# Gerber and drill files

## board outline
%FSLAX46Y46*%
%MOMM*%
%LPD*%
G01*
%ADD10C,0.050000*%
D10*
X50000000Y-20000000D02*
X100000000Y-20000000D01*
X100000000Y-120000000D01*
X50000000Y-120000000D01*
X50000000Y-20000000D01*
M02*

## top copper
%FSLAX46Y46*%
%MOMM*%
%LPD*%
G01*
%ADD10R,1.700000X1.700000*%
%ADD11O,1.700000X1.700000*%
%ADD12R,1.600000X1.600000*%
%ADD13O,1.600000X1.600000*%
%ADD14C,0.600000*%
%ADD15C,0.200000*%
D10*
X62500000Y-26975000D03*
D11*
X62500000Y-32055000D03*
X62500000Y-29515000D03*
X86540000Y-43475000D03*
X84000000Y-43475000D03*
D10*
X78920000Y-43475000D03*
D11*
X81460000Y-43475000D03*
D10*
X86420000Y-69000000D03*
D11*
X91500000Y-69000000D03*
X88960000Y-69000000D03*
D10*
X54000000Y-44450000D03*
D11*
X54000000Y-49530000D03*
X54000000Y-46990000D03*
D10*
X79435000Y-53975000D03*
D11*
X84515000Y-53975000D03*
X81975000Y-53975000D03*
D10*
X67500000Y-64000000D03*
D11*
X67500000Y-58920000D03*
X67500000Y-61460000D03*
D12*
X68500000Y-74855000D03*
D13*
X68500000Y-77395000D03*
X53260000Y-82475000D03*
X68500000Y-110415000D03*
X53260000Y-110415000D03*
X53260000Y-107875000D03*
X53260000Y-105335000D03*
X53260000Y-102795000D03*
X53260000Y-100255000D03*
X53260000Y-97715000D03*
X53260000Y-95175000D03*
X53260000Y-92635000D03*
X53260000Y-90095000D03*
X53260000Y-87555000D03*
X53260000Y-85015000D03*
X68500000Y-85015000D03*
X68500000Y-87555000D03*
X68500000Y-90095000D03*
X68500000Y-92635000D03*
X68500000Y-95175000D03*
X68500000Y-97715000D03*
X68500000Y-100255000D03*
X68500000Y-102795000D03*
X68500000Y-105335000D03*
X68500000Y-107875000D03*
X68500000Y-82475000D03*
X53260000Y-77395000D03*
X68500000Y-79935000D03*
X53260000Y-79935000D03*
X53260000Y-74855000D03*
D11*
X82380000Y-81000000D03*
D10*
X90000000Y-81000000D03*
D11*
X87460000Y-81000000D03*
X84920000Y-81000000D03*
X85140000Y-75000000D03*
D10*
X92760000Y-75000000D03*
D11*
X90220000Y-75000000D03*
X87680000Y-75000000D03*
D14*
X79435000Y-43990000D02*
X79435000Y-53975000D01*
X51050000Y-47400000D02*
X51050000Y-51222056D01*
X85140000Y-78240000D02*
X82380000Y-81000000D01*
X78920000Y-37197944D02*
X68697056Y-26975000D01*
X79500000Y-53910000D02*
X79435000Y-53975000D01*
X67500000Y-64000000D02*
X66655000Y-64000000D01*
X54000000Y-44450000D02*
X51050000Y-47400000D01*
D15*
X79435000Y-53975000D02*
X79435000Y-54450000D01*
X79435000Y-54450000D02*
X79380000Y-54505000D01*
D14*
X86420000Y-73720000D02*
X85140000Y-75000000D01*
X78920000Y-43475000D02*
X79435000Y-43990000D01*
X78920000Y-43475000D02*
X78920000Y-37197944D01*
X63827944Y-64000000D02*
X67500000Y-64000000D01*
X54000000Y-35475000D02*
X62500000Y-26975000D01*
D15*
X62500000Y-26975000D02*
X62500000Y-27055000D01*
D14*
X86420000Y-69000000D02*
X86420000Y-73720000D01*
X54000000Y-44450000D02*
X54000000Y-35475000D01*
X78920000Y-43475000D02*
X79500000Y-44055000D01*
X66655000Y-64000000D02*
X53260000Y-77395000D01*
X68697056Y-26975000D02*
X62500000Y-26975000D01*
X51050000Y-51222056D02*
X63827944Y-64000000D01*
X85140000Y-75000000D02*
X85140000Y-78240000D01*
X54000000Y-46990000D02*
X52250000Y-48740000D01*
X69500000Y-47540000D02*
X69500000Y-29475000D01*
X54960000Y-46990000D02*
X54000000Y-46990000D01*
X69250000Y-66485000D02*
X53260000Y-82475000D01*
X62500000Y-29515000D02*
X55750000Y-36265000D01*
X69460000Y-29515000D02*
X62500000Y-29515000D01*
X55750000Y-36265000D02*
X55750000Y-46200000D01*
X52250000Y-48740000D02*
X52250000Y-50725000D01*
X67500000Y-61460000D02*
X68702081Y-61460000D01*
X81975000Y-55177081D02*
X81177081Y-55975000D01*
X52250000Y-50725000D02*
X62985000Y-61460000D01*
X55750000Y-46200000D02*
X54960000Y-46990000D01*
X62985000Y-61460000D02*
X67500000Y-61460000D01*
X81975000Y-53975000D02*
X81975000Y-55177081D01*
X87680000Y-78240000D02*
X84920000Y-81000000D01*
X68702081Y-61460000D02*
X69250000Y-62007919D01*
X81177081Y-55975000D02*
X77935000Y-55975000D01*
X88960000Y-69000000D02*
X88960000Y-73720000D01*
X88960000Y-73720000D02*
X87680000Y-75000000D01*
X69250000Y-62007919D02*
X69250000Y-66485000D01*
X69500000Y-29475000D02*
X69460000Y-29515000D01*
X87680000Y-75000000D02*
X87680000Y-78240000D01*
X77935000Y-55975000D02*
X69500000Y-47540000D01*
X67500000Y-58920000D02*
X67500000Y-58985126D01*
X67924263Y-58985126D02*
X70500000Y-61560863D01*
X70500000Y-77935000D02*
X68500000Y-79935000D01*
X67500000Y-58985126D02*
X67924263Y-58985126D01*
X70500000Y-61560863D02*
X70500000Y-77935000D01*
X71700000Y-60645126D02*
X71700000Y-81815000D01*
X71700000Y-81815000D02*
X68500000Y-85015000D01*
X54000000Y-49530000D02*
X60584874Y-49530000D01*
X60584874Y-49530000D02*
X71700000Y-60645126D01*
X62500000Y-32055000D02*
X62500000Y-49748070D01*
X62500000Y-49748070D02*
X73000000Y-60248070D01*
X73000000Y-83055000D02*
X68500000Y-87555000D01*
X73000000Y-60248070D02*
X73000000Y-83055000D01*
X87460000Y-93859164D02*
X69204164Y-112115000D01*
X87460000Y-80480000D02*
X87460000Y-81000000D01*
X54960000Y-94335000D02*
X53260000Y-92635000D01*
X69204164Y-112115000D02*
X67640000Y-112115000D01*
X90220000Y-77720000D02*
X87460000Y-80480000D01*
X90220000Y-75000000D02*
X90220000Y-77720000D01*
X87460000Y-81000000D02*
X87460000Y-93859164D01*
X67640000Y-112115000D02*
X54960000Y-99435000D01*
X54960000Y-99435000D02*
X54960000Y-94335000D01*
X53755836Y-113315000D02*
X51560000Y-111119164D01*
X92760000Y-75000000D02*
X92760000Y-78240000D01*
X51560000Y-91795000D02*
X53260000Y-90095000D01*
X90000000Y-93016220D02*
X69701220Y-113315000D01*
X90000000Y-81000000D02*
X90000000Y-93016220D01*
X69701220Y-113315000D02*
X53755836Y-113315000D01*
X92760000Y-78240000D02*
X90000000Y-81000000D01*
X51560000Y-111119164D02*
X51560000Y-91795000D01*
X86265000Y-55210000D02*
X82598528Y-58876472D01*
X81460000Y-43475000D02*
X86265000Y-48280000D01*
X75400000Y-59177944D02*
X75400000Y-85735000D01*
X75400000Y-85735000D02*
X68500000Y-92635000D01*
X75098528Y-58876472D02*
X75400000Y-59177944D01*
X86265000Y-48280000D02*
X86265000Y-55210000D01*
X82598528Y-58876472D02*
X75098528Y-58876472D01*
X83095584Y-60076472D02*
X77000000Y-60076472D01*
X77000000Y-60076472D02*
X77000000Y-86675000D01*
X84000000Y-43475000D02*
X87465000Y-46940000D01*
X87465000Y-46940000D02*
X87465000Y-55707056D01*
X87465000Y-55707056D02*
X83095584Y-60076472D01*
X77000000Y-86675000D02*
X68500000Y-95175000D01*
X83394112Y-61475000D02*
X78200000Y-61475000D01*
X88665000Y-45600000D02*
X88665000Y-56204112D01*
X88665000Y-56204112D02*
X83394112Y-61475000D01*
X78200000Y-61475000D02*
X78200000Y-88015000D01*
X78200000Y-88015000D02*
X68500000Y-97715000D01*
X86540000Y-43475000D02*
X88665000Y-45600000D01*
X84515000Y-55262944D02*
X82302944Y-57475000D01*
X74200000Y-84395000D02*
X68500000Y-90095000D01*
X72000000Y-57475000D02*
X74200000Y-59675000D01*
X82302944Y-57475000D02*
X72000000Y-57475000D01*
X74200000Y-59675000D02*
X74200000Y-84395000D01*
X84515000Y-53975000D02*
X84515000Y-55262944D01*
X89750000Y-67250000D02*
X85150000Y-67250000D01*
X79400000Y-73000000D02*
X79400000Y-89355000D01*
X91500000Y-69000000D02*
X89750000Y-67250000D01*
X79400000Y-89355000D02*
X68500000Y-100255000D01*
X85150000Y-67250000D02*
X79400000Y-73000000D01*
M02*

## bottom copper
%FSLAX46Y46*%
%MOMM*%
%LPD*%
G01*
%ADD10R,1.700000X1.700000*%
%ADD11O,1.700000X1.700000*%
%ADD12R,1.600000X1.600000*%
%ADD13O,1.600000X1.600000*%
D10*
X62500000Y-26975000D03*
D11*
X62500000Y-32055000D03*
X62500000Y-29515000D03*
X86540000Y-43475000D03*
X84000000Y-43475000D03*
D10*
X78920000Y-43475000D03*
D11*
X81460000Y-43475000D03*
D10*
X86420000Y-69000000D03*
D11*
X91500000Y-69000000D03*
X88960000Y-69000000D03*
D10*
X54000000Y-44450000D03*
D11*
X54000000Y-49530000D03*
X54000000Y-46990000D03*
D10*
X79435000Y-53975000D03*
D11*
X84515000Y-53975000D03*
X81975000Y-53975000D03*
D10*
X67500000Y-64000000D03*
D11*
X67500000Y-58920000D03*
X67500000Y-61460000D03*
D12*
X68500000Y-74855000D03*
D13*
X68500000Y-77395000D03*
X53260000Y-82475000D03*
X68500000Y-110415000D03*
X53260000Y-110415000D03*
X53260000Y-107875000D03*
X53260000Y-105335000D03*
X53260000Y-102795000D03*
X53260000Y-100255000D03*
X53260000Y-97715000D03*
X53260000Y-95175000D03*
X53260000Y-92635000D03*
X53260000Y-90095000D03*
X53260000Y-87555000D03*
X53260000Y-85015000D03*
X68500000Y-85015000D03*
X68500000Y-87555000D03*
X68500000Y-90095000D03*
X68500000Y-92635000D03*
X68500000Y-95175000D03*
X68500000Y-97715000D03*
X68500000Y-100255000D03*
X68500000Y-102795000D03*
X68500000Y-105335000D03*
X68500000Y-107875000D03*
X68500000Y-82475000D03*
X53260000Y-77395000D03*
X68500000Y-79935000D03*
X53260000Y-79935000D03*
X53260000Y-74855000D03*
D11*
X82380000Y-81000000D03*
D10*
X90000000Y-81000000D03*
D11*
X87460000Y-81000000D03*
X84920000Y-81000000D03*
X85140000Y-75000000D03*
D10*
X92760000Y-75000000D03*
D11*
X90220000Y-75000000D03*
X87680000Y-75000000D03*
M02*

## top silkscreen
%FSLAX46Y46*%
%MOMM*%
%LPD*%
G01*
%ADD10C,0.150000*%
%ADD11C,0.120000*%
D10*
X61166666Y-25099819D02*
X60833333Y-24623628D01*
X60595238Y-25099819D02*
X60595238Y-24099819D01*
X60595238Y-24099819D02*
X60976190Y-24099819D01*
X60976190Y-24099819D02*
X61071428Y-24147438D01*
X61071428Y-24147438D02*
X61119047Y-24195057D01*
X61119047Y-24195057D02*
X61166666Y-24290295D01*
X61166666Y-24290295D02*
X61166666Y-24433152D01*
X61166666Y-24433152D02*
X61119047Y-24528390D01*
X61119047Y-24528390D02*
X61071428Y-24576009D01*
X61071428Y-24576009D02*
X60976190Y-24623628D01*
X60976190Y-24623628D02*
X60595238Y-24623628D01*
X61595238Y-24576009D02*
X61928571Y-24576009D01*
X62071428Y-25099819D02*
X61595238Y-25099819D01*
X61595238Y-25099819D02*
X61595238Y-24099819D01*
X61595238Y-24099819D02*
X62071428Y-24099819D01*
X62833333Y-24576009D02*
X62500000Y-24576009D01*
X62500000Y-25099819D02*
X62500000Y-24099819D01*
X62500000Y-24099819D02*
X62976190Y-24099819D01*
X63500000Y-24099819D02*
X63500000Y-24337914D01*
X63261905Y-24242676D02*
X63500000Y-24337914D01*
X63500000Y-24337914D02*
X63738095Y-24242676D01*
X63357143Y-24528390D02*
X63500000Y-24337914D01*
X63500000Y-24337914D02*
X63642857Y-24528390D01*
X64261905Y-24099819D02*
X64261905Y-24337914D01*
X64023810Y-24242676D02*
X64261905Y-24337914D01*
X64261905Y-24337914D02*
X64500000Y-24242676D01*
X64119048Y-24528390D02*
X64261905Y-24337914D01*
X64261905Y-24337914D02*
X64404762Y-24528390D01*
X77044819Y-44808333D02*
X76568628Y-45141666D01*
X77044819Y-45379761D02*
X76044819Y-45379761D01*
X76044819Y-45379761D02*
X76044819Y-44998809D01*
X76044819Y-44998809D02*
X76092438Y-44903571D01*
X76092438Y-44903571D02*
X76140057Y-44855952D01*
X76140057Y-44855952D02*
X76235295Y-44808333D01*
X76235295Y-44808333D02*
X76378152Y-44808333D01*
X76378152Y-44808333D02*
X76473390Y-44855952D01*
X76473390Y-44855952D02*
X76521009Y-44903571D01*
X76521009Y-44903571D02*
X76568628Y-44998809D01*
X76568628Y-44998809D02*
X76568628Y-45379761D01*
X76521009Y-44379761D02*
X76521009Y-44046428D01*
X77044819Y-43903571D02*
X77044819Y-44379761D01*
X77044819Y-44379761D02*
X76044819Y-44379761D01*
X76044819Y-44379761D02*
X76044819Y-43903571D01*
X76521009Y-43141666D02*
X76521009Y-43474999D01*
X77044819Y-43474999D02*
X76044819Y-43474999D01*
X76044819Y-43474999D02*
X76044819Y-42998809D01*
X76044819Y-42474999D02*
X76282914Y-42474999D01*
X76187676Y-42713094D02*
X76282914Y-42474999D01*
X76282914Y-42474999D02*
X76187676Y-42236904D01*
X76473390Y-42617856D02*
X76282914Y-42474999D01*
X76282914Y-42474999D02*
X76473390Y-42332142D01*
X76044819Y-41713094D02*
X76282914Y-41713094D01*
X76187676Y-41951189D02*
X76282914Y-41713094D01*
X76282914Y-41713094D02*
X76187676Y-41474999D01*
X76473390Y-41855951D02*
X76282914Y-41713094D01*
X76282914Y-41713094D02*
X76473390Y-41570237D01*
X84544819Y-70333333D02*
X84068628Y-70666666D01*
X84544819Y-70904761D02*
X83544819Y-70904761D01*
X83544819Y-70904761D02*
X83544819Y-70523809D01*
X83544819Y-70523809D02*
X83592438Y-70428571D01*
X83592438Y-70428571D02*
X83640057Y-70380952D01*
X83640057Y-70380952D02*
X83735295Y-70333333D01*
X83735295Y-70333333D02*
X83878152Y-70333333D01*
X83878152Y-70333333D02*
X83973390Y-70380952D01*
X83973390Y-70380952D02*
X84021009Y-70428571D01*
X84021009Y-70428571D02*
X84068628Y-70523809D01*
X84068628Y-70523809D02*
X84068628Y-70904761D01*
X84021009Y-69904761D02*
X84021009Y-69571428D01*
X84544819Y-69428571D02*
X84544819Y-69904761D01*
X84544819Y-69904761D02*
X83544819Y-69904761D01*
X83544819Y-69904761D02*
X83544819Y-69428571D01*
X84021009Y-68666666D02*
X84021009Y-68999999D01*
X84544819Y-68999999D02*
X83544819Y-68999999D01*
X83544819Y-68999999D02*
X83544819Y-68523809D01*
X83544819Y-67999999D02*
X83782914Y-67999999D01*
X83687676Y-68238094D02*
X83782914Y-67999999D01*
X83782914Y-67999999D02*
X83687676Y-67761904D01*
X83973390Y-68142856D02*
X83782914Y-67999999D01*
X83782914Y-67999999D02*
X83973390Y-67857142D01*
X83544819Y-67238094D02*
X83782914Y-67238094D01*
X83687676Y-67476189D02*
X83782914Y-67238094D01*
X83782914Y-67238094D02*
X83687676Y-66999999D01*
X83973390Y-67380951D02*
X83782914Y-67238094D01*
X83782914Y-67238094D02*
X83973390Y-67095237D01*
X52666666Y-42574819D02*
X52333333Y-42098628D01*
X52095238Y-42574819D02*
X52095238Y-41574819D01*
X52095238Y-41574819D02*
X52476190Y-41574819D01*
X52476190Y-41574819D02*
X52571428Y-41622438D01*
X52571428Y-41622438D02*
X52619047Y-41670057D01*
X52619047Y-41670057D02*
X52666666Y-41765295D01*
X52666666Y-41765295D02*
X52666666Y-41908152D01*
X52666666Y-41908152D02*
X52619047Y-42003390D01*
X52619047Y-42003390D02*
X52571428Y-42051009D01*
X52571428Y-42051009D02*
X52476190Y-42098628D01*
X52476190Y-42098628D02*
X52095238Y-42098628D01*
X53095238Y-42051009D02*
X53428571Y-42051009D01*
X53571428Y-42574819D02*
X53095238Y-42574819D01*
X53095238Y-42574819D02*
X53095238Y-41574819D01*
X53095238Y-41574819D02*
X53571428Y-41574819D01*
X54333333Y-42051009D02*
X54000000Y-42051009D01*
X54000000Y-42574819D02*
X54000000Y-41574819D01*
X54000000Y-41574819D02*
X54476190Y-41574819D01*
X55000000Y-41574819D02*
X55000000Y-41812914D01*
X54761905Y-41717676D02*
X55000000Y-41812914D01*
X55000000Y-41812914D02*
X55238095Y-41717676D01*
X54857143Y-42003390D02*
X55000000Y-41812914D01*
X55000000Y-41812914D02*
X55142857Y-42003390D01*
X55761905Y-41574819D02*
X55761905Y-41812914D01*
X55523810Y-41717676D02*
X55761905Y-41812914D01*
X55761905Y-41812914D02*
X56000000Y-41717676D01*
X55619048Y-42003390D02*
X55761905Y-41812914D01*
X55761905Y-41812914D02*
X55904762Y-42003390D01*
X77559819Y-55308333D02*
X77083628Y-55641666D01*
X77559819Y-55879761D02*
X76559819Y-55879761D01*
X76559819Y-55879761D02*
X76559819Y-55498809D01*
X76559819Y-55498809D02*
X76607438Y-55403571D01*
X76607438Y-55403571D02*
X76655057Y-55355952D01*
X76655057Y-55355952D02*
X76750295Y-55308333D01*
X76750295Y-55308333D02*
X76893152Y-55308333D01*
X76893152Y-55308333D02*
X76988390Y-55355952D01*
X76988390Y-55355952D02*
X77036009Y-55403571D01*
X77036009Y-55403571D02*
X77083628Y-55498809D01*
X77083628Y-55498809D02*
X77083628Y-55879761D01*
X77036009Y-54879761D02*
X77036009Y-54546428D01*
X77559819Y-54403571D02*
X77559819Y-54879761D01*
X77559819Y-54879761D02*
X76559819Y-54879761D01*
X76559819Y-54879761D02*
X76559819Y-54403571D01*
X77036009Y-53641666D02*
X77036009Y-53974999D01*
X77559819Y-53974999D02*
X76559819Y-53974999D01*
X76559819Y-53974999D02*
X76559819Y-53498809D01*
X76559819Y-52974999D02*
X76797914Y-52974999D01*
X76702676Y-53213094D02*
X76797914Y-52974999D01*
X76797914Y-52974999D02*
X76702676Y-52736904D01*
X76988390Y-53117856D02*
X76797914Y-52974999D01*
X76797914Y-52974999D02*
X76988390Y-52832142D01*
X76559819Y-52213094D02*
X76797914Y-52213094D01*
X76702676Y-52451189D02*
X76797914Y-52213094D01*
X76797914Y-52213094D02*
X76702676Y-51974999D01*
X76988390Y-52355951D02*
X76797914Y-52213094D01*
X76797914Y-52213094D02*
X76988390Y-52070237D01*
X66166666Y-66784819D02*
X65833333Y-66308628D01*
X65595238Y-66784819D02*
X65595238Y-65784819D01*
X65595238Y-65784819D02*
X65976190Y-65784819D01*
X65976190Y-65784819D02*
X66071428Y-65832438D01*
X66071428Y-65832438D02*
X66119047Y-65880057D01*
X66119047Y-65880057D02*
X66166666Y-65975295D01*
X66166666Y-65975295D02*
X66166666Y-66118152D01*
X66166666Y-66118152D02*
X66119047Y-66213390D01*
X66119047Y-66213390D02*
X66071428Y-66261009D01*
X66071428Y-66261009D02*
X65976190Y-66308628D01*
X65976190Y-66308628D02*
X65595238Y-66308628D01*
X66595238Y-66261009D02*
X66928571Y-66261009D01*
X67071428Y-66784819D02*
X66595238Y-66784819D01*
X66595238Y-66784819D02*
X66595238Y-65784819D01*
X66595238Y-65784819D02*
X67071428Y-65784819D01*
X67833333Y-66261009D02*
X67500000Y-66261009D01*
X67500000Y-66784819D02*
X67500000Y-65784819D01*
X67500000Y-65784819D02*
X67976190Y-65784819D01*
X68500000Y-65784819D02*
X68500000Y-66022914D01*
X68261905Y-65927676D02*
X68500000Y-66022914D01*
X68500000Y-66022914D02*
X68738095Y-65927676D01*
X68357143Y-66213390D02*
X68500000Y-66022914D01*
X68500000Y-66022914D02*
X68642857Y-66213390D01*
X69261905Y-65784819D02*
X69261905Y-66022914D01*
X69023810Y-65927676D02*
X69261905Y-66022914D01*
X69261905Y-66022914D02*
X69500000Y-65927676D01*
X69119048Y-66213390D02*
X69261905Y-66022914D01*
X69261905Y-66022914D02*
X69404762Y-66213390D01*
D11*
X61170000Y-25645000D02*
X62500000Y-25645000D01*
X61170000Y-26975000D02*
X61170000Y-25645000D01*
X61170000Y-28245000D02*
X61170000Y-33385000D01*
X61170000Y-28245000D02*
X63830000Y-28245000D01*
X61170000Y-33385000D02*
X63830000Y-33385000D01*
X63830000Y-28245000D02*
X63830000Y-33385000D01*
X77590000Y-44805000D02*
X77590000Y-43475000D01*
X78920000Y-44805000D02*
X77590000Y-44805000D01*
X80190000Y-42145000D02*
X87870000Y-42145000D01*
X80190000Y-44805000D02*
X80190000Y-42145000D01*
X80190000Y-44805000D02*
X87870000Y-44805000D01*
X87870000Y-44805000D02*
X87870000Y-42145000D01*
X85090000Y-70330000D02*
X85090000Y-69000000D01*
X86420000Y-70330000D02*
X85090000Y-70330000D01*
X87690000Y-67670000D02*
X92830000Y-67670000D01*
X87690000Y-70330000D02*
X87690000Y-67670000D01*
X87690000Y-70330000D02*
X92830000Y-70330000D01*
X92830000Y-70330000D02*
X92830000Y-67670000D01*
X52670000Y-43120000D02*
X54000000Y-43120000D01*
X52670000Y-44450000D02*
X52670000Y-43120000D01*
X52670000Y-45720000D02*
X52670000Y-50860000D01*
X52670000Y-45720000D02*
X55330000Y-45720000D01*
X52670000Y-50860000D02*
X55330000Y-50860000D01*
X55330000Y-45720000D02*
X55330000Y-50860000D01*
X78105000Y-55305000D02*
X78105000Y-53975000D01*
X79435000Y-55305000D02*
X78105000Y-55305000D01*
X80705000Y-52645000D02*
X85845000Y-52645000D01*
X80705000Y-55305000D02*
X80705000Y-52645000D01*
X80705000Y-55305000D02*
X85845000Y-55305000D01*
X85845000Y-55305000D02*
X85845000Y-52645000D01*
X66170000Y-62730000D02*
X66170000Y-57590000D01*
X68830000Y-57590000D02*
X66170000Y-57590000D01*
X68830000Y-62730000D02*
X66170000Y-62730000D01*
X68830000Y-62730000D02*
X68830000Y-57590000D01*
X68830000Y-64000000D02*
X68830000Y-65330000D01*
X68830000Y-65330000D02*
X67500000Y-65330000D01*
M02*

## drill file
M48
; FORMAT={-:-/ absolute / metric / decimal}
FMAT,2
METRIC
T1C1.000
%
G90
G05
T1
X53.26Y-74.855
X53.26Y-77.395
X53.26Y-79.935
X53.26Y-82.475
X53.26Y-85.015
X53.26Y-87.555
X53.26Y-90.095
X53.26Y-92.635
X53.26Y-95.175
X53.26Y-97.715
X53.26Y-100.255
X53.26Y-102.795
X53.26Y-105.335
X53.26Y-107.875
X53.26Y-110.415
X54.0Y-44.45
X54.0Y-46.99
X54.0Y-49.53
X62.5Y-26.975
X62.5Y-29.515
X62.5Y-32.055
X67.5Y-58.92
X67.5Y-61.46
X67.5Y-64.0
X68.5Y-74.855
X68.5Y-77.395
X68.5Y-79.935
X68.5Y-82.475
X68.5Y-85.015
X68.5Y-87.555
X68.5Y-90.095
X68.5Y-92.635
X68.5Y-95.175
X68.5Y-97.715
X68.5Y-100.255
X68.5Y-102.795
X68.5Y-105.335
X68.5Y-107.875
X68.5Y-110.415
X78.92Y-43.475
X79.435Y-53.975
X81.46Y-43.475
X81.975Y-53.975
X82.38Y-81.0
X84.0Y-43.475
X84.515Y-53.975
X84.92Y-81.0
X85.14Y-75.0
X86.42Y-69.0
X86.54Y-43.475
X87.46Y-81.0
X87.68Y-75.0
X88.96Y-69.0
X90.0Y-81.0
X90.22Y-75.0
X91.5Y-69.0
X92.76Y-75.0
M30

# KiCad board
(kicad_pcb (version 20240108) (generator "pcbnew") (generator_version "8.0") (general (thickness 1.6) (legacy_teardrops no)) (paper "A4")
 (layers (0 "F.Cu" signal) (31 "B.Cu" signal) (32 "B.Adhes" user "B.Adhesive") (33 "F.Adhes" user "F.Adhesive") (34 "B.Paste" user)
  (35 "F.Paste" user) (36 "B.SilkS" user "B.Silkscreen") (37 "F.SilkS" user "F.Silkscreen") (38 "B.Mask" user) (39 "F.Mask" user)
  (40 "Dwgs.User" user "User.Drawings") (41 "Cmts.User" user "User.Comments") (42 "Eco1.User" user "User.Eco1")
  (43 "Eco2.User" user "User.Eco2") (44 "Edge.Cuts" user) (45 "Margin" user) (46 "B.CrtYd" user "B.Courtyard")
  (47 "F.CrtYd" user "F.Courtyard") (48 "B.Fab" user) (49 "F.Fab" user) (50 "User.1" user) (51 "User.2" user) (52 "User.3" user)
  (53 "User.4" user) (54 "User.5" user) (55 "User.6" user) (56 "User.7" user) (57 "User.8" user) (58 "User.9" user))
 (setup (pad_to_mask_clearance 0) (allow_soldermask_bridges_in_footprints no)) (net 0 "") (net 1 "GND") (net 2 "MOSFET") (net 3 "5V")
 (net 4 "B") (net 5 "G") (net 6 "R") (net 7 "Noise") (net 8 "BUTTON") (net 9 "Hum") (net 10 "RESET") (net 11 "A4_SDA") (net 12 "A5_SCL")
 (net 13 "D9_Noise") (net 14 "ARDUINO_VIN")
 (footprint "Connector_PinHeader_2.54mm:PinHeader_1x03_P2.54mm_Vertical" (layer "F.Cu") (at 62.5 26.975)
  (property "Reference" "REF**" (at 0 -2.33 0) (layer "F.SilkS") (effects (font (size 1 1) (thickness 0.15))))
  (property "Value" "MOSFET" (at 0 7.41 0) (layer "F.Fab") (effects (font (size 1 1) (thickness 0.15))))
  (fp_line (start -1.33 -1.33) (end 0 -1.33) (stroke (width 0.12) (type solid)) (layer "F.SilkS"))
  (fp_line (start -1.33 0) (end -1.33 -1.33) (stroke (width 0.12) (type solid)) (layer "F.SilkS"))
  (fp_line (start -1.33 1.27) (end -1.33 6.41) (stroke (width 0.12) (type solid)) (layer "F.SilkS"))
  (fp_line (start -1.33 1.27) (end 1.33 1.27) (stroke (width 0.12) (type solid)) (layer "F.SilkS"))
  (fp_line (start -1.33 6.41) (end 1.33 6.41) (stroke (width 0.12) (type solid)) (layer "F.SilkS"))
  (fp_line (start 1.33 1.27) (end 1.33 6.41) (stroke (width 0.12) (type solid)) (layer "F.SilkS"))
  (pad "GND" thru_hole rect (at 0 0) (size 1.7 1.7) (drill 1) (layers "*.Cu" "*.Mask") (remove_unused_layers no) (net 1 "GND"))
  (pad "S" thru_hole oval (at 0 5.08) (size 1.7 1.7) (drill 1) (layers "*.Cu" "*.Mask") (remove_unused_layers no) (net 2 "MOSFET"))
  (pad "VCC" thru_hole oval (at 0 2.54) (size 1.7 1.7) (drill 1) (layers "*.Cu" "*.Mask") (remove_unused_layers no) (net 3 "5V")))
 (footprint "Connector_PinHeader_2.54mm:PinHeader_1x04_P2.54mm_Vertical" (layer "F.Cu") (at 78.92 43.475 90)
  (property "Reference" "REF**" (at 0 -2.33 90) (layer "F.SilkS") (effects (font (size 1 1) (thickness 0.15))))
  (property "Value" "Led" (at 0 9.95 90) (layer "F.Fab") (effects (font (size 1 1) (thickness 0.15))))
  (fp_line (start -1.33 -1.33) (end 0 -1.33) (stroke (width 0.12) (type solid)) (layer "F.SilkS"))
  (fp_line (start -1.33 0) (end -1.33 -1.33) (stroke (width 0.12) (type solid)) (layer "F.SilkS"))
  (fp_line (start 1.33 1.27) (end 1.33 8.95) (stroke (width 0.12) (type solid)) (layer "F.SilkS"))
  (fp_line (start -1.33 1.27) (end 1.33 1.27) (stroke (width 0.12) (type solid)) (layer "F.SilkS"))
  (fp_line (start -1.33 1.27) (end -1.33 8.95) (stroke (width 0.12) (type solid)) (layer "F.SilkS"))
  (fp_line (start -1.33 8.95) (end 1.33 8.95) (stroke (width 0.12) (type solid)) (layer "F.SilkS"))
  (pad "B" thru_hole oval (at 0 7.62 90) (size 1.7 1.7) (drill 1) (layers "*.Cu" "*.Mask") (remove_unused_layers no) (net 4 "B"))
  (pad "G" thru_hole oval (at 0 5.08 90) (size 1.7 1.7) (drill 1) (layers "*.Cu" "*.Mask") (remove_unused_layers no) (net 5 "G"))
  (pad "GND" thru_hole rect (at 0 0 90) (size 1.7 1.7) (drill 1) (layers "*.Cu" "*.Mask") (remove_unused_layers no) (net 1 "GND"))
  (pad "R" thru_hole oval (at 0 2.54 90) (size 1.7 1.7) (drill 1) (layers "*.Cu" "*.Mask") (remove_unused_layers no) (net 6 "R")))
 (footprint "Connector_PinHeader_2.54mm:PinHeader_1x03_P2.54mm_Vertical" (layer "F.Cu") (at 86.42 69 90)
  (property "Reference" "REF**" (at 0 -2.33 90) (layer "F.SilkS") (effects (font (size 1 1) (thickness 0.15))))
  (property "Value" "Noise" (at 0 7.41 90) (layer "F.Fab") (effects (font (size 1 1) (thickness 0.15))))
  (fp_line (start -1.33 -1.33) (end 0 -1.33) (stroke (width 0.12) (type solid)) (layer "F.SilkS"))
  (fp_line (start -1.33 0) (end -1.33 -1.33) (stroke (width 0.12) (type solid)) (layer "F.SilkS"))
  (fp_line (start 1.33 1.27) (end 1.33 6.41) (stroke (width 0.12) (type solid)) (layer "F.SilkS"))
  (fp_line (start -1.33 1.27) (end 1.33 1.27) (stroke (width 0.12) (type solid)) (layer "F.SilkS"))
  (fp_line (start -1.33 1.27) (end -1.33 6.41) (stroke (width 0.12) (type solid)) (layer "F.SilkS"))
  (fp_line (start -1.33 6.41) (end 1.33 6.41) (stroke (width 0.12) (type solid)) (layer "F.SilkS"))
  (pad "GND" thru_hole rect (at 0 0 90) (size 1.7 1.7) (drill 1) (layers "*.Cu" "*.Mask") (remove_unused_layers no) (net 1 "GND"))
  (pad "S" thru_hole oval (at 0 5.08 90) (size 1.7 1.7) (drill 1) (layers "*.Cu" "*.Mask") (remove_unused_layers no) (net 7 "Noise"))
  (pad "VCC" thru_hole oval (at 0 2.54 90) (size 1.7 1.7) (drill 1) (layers "*.Cu" "*.Mask") (remove_unused_layers no) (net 3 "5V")))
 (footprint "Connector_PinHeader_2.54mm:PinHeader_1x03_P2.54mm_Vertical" (layer "F.Cu") (at 54 44.45)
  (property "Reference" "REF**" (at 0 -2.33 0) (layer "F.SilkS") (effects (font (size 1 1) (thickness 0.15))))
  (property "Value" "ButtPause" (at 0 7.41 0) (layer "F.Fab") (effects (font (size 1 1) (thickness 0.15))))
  (fp_line (start -1.33 -1.33) (end 0 -1.33) (stroke (width 0.12) (type solid)) (layer "F.SilkS"))
  (fp_line (start -1.33 0) (end -1.33 -1.33) (stroke (width 0.12) (type solid)) (layer "F.SilkS"))
  (fp_line (start -1.33 1.27) (end -1.33 6.41) (stroke (width 0.12) (type solid)) (layer "F.SilkS"))
  (fp_line (start -1.33 1.27) (end 1.33 1.27) (stroke (width 0.12) (type solid)) (layer "F.SilkS"))
  (fp_line (start -1.33 6.41) (end 1.33 6.41) (stroke (width 0.12) (type solid)) (layer "F.SilkS"))
  (fp_line (start 1.33 1.27) (end 1.33 6.41) (stroke (width 0.12) (type solid)) (layer "F.SilkS"))
  (pad "GND" thru_hole rect (at 0 0) (size 1.7 1.7) (drill 1) (layers "*.Cu" "*.Mask") (remove_unused_layers no) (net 1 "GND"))
  (pad "S" thru_hole oval (at 0 5.08) (size 1.7 1.7) (drill 1) (layers "*.Cu" "*.Mask") (remove_unused_layers no) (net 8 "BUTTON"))
  (pad "VCC" thru_hole oval (at 0 2.54) (size 1.7 1.7) (drill 1) (layers "*.Cu" "*.Mask") (remove_unused_layers no) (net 3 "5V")))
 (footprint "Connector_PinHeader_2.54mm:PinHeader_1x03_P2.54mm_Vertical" (layer "F.Cu") (at 79.435 53.975 90)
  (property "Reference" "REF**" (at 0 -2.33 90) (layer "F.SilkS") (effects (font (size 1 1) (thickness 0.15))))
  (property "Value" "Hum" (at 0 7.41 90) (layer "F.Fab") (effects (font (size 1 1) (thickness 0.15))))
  (fp_line (start -1.33 -1.33) (end 0 -1.33) (stroke (width 0.12) (type solid)) (layer "F.SilkS"))
  (fp_line (start -1.33 0) (end -1.33 -1.33) (stroke (width 0.12) (type solid)) (layer "F.SilkS"))
  (fp_line (start 1.33 1.27) (end 1.33 6.41) (stroke (width 0.12) (type solid)) (layer "F.SilkS"))
  (fp_line (start -1.33 1.27) (end 1.33 1.27) (stroke (width 0.12) (type solid)) (layer "F.SilkS"))
  (fp_line (start -1.33 1.27) (end -1.33 6.41) (stroke (width 0.12) (type solid)) (layer "F.SilkS"))
  (fp_line (start -1.33 6.41) (end 1.33 6.41) (stroke (width 0.12) (type solid)) (layer "F.SilkS"))
  (pad "GND" thru_hole rect (at 0 0 90) (size 1.7 1.7) (drill 1) (layers "*.Cu" "*.Mask") (remove_unused_layers no) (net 1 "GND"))
  (pad "S" thru_hole oval (at 0 5.08 90) (size 1.7 1.7) (drill 1) (layers "*.Cu" "*.Mask") (remove_unused_layers no) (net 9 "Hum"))
  (pad "VCC" thru_hole oval (at 0 2.54 90) (size 1.7 1.7) (drill 1) (layers "*.Cu" "*.Mask") (remove_unused_layers no) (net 3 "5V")))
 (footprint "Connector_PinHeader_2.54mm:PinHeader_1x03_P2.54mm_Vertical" (layer "F.Cu") (at 67.5 64 180)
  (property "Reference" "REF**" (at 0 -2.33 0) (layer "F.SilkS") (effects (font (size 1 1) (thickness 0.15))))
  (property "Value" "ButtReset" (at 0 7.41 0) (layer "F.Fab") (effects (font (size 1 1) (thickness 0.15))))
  (fp_line (start 1.33 1.27) (end 1.33 6.41) (stroke (width 0.12) (type solid)) (layer "F.SilkS"))
  (fp_line (start -1.33 6.41) (end 1.33 6.41) (stroke (width 0.12) (type solid)) (layer "F.SilkS"))
  (fp_line (start -1.33 1.27) (end 1.33 1.27) (stroke (width 0.12) (type solid)) (layer "F.SilkS"))
  (fp_line (start -1.33 1.27) (end -1.33 6.41) (stroke (width 0.12) (type solid)) (layer "F.SilkS"))
  (fp_line (start -1.33 0) (end -1.33 -1.33) (stroke (width 0.12) (type solid)) (layer "F.SilkS"))
  (fp_line (start -1.33 -1.33) (end 0 -1.33) (stroke (width 0.12) (type solid)) (layer "F.SilkS"))
  (pad "GND" thru_hole rect (at 0 0 180) (size 1.7 1.7) (drill 1) (layers "*.Cu" "*.Mask") (remove_unused_layers no) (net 1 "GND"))
  (pad "S" thru_hole oval (at 0 5.08 180) (size 1.7 1.7) (drill 1) (layers "*.Cu" "*.Mask") (remove_unused_layers no) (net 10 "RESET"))
  (pad "VCC" thru_hole oval (at 0 2.54 180) (size 1.7 1.7) (drill 1) (layers "*.Cu" "*.Mask") (remove_unused_layers no) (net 3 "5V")))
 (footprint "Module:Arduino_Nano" (layer "B.Cu") (at 68.5 74.855 180)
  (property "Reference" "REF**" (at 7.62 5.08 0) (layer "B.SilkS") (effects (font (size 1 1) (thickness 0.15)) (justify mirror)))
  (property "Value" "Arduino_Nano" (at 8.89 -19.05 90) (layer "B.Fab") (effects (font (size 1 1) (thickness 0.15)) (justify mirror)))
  (pad "1" thru_hole rect (at 0 0 180) (size 1.6 1.6) (drill 1) (layers "*.Cu" "*.Mask") (remove_unused_layers no))
  (pad "2" thru_hole oval (at 0 -2.54 180) (size 1.6 1.6) (drill 1) (layers "*.Cu" "*.Mask") (remove_unused_layers no))
  (pad "5V" thru_hole oval (at 15.24 -7.62 180) (size 1.6 1.6) (drill 1) (layers "*.Cu" "*.Mask") (remove_unused_layers no) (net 3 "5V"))
  (pad "15" thru_hole oval (at 0 -35.56 180) (size 1.6 1.6) (drill 1) (layers "*.Cu" "*.Mask") (remove_unused_layers no))
  (pad "16" thru_hole oval (at 15.24 -35.56 180) (size 1.6 1.6) (drill 1) (layers "*.Cu" "*.Mask") (remove_unused_layers no))
  (pad "17" thru_hole oval (at 15.24 -33.02 180) (size 1.6 1.6) (drill 1) (layers "*.Cu" "*.Mask") (remove_unused_layers no))
  (pad "18" thru_hole oval (at 15.24 -30.48 180) (size 1.6 1.6) (drill 1) (layers "*.Cu" "*.Mask") (remove_unused_layers no))
  (pad "A0" thru_hole oval (at 15.24 -27.94 180) (size 1.6 1.6) (drill 1) (layers "*.Cu" "*.Mask") (remove_unused_layers no))
  (pad "A1" thru_hole oval (at 15.24 -25.4 180) (size 1.6 1.6) (drill 1) (layers "*.Cu" "*.Mask") (remove_unused_layers no))
  (pad "A2" thru_hole oval (at 15.24 -22.86 180) (size 1.6 1.6) (drill 1) (layers "*.Cu" "*.Mask") (remove_unused_layers no))
  (pad "A3" thru_hole oval (at 15.24 -20.32 180) (size 1.6 1.6) (drill 1) (layers "*.Cu" "*.Mask") (remove_unused_layers no))
  (pad "A4" thru_hole oval (at 15.24 -17.78 180) (size 1.6 1.6) (drill 1) (layers "*.Cu" "*.Mask") (remove_unused_layers no)
   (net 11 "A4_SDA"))
  (pad "A5" thru_hole oval (at 15.24 -15.24 180) (size 1.6 1.6) (drill 1) (layers "*.Cu" "*.Mask") (remove_unused_layers no)
   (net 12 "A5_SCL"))
  (pad "A6" thru_hole oval (at 15.24 -12.7 180) (size 1.6 1.6) (drill 1) (layers "*.Cu" "*.Mask") (remove_unused_layers no))
  (pad "A7" thru_hole oval (at 15.24 -10.16 180) (size 1.6 1.6) (drill 1) (layers "*.Cu" "*.Mask") (remove_unused_layers no))
  (pad "D2" thru_hole oval (at 0 -10.16 180) (size 1.6 1.6) (drill 1) (layers "*.Cu" "*.Mask") (remove_unused_layers no) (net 8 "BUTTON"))
  (pad "D3" thru_hole oval (at 0 -12.7 180) (size 1.6 1.6) (drill 1) (layers "*.Cu" "*.Mask") (remove_unused_layers no) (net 2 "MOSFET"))
  (pad "D4" thru_hole oval (at 0 -15.24 180) (size 1.6 1.6) (drill 1) (layers "*.Cu" "*.Mask") (remove_unused_layers no) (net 9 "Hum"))
  (pad "D5" thru_hole oval (at 0 -17.78 180) (size 1.6 1.6) (drill 1) (layers "*.Cu" "*.Mask") (remove_unused_layers no) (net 6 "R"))
  (pad "D6" thru_hole oval (at 0 -20.32 180) (size 1.6 1.6) (drill 1) (layers "*.Cu" "*.Mask") (remove_unused_layers no) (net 5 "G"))
  (pad "D7" thru_hole oval (at 0 -22.86 180) (size 1.6 1.6) (drill 1) (layers "*.Cu" "*.Mask") (remove_unused_layers no) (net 4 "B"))
  (pad "D8" thru_hole oval (at 0 -25.4 180) (size 1.6 1.6) (drill 1) (layers "*.Cu" "*.Mask") (remove_unused_layers no) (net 7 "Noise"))
  (pad "D9" thru_hole oval (at 0 -27.94 180) (size 1.6 1.6) (drill 1) (layers "*.Cu" "*.Mask") (remove_unused_layers no) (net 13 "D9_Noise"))
  (pad "D10" thru_hole oval (at 0 -30.48 180) (size 1.6 1.6) (drill 1) (layers "*.Cu" "*.Mask") (remove_unused_layers no))
  (pad "D11" thru_hole oval (at 0 -33.02 180) (size 1.6 1.6) (drill 1) (layers "*.Cu" "*.Mask") (remove_unused_layers no))
  (pad "GND" thru_hole oval (at 0 -7.62 180) (size 1.6 1.6) (drill 1) (layers "*.Cu" "*.Mask") (remove_unused_layers no) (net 1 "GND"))
  (pad "GND" thru_hole oval (at 15.24 -2.54 180) (size 1.6 1.6) (drill 1) (layers "*.Cu" "*.Mask") (remove_unused_layers no) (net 1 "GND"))
  (pad "RST" thru_hole oval (at 0 -5.08 180) (size 1.6 1.6) (drill 1) (layers "*.Cu" "*.Mask") (remove_unused_layers no) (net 10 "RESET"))
  (pad "RST" thru_hole oval (at 15.24 -5.08 180) (size 1.6 1.6) (drill 1) (layers "*.Cu" "*.Mask") (remove_unused_layers no))
  (pad "VIN" thru_hole oval (at 15.24 0 180) (size 1.6 1.6) (drill 1) (layers "*.Cu" "*.Mask") (remove_unused_layers no)
   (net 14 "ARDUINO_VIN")))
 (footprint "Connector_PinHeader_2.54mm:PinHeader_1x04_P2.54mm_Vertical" (layer "B.Cu") (at 90 81 90)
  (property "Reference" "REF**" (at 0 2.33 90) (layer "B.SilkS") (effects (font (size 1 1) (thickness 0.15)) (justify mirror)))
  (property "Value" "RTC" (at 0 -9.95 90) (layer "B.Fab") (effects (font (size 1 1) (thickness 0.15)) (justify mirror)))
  (pad "GND" thru_hole oval (at 0 -7.62 90) (size 1.7 1.7) (drill 1) (layers "*.Cu" "*.Mask") (remove_unused_layers no) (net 1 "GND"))
  (pad "SCL" thru_hole rect (at 0 0 90) (size 1.7 1.7) (drill 1) (layers "*.Cu" "*.Mask") (remove_unused_layers no) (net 12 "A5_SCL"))
  (pad "SDA" thru_hole oval (at 0 -2.54 90) (size 1.7 1.7) (drill 1) (layers "*.Cu" "*.Mask") (remove_unused_layers no) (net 11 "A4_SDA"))
  (pad "VCC" thru_hole oval (at 0 -5.08 90) (size 1.7 1.7) (drill 1) (layers "*.Cu" "*.Mask") (remove_unused_layers no) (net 3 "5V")))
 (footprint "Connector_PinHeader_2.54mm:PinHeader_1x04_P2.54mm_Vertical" (layer "B.Cu") (at 92.76 75 90)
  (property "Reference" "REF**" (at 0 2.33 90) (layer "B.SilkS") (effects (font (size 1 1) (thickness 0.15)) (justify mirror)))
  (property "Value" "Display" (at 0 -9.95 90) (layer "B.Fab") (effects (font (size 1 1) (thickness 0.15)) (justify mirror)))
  (pad "GND" thru_hole oval (at 0 -7.62 90) (size 1.7 1.7) (drill 1) (layers "*.Cu" "*.Mask") (remove_unused_layers no) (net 1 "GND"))
  (pad "SCL" thru_hole rect (at 0 0 90) (size 1.7 1.7) (drill 1) (layers "*.Cu" "*.Mask") (remove_unused_layers no) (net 12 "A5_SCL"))
  (pad "SDA" thru_hole oval (at 0 -2.54 90) (size 1.7 1.7) (drill 1) (layers "*.Cu" "*.Mask") (remove_unused_layers no) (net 11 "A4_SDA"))
  (pad "VCC" thru_hole oval (at 0 -5.08 90) (size 1.7 1.7) (drill 1) (layers "*.Cu" "*.Mask") (remove_unused_layers no) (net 3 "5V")))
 (gr_rect (start 50 20) (end 100 120) (stroke (width 0.05) (type default)) (fill none) (layer "Edge.Cuts"))
 (segment (start 79.435 43.99) (end 79.435 53.975) (width 0.6) (layer "F.Cu") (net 1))
 (segment (start 51.05 47.4) (end 51.05 51.222056) (width 0.6) (layer "F.Cu") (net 1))
 (segment (start 85.14 78.24) (end 82.38 81) (width 0.6) (layer "F.Cu") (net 1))
 (segment (start 78.92 37.197944) (end 68.697056 26.975) (width 0.6) (layer "F.Cu") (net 1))
 (segment (start 79.5 53.91) (end 79.435 53.975) (width 0.6) (layer "F.Cu") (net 1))
 (segment (start 67.5 64) (end 66.655 64) (width 0.6) (layer "F.Cu") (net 1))
 (segment (start 54 44.45) (end 51.05 47.4) (width 0.6) (layer "F.Cu") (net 1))
 (segment (start 79.435 53.975) (end 79.435 54.45) (width 0.2) (layer "F.Cu") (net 1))
 (segment (start 79.435 54.45) (end 79.38 54.505) (width 0.2) (layer "F.Cu") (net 1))
 (segment (start 86.42 73.72) (end 85.14 75) (width 0.6) (layer "F.Cu") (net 1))
 (segment (start 78.92 43.475) (end 79.435 43.99) (width 0.6) (layer "F.Cu") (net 1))
 (segment (start 78.92 43.475) (end 78.92 37.197944) (width 0.6) (layer "F.Cu") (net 1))
 (segment (start 63.827944 64) (end 67.5 64) (width 0.6) (layer "F.Cu") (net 1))
 (segment (start 54 35.475) (end 62.5 26.975) (width 0.6) (layer "F.Cu") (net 1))
 (segment (start 62.5 26.975) (end 62.5 27.055) (width 0.2) (layer "F.Cu") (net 1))
 (segment (start 86.42 69) (end 86.42 73.72) (width 0.6) (layer "F.Cu") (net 1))
 (segment (start 54 44.45) (end 54 35.475) (width 0.6) (layer "F.Cu") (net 1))
 (segment (start 78.92 43.475) (end 79.5 44.055) (width 0.6) (layer "F.Cu") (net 1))
 (segment (start 66.655 64) (end 53.26 77.395) (width 0.6) (layer "F.Cu") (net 1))
 (segment (start 68.697056 26.975) (end 62.5 26.975) (width 0.6) (layer "F.Cu") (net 1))
 (segment (start 51.05 51.222056) (end 63.827944 64) (width 0.6) (layer "F.Cu") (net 1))
 (segment (start 85.14 75) (end 85.14 78.24) (width 0.6) (layer "F.Cu") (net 1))
 (segment (start 54 46.99) (end 52.25 48.74) (width 0.6) (layer "F.Cu") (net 3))
 (segment (start 69.5 47.54) (end 69.5 29.475) (width 0.6) (layer "F.Cu") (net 3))
 (segment (start 54.96 46.99) (end 54 46.99) (width 0.6) (layer "F.Cu") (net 3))
 (segment (start 69.25 66.485) (end 53.26 82.475) (width 0.6) (layer "F.Cu") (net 3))
 (segment (start 62.5 29.515) (end 55.75 36.265) (width 0.6) (layer "F.Cu") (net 3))
 (segment (start 69.46 29.515) (end 62.5 29.515) (width 0.6) (layer "F.Cu") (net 3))
 (segment (start 55.75 36.265) (end 55.75 46.2) (width 0.6) (layer "F.Cu") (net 3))
 (segment (start 52.25 48.74) (end 52.25 50.725) (width 0.6) (layer "F.Cu") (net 3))
 (segment (start 67.5 61.46) (end 68.702081 61.46) (width 0.6) (layer "F.Cu") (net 3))
 (segment (start 81.975 55.177081) (end 81.177081 55.975) (width 0.6) (layer "F.Cu") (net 3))
 (segment (start 52.25 50.725) (end 62.985 61.46) (width 0.6) (layer "F.Cu") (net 3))
 (segment (start 55.75 46.2) (end 54.96 46.99) (width 0.6) (layer "F.Cu") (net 3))
 (segment (start 62.985 61.46) (end 67.5 61.46) (width 0.6) (layer "F.Cu") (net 3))
 (segment (start 81.975 53.975) (end 81.975 55.177081) (width 0.6) (layer "F.Cu") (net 3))
 (segment (start 87.68 78.24) (end 84.92 81) (width 0.6) (layer "F.Cu") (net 3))
 (segment (start 68.702081 61.46) (end 69.25 62.007919) (width 0.6) (layer "F.Cu") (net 3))
 (segment (start 81.177081 55.975) (end 77.935 55.975) (width 0.6) (layer "F.Cu") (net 3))
 (segment (start 88.96 69) (end 88.96 73.72) (width 0.6) (layer "F.Cu") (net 3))
 (segment (start 88.96 73.72) (end 87.68 75) (width 0.6) (layer "F.Cu") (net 3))
 (segment (start 69.25 62.007919) (end 69.25 66.485) (width 0.6) (layer "F.Cu") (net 3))
 (segment (start 69.5 29.475) (end 69.46 29.515) (width 0.6) (layer "F.Cu") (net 3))
 (segment (start 87.68 75) (end 87.68 78.24) (width 0.6) (layer "F.Cu") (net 3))
 (segment (start 77.935 55.975) (end 69.5 47.54) (width 0.6) (layer "F.Cu") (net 3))
 (segment (start 67.5 58.92) (end 67.5 58.985126) (width 0.6) (layer "F.Cu") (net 10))
 (segment (start 67.924263 58.985126) (end 70.5 61.560863) (width 0.6) (layer "F.Cu") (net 10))
 (segment (start 70.5 77.935) (end 68.5 79.935) (width 0.6) (layer "F.Cu") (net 10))
 (segment (start 67.5 58.985126) (end 67.924263 58.985126) (width 0.6) (layer "F.Cu") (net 10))
 (segment (start 70.5 61.560863) (end 70.5 77.935) (width 0.6) (layer "F.Cu") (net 10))
 (segment (start 71.7 60.645126) (end 71.7 81.815) (width 0.6) (layer "F.Cu") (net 8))
 (segment (start 71.7 81.815) (end 68.5 85.015) (width 0.6) (layer "F.Cu") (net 8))
 (segment (start 54 49.53) (end 60.584874 49.53) (width 0.6) (layer "F.Cu") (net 8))
 (segment (start 60.584874 49.53) (end 71.7 60.645126) (width 0.6) (layer "F.Cu") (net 8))
 (segment (start 62.5 32.055) (end 62.5 49.74807) (width 0.6) (layer "F.Cu") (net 2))
 (segment (start 62.5 49.74807) (end 73 60.24807) (width 0.6) (layer "F.Cu") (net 2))
 (segment (start 73 83.055) (end 68.5 87.555) (width 0.6) (layer "F.Cu") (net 2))
 (segment (start 73 60.24807) (end 73 83.055) (width 0.6) (layer "F.Cu") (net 2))
 (segment (start 87.46 93.859164) (end 69.204164 112.115) (width 0.6) (layer "F.Cu") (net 11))
 (segment (start 87.46 80.48) (end 87.46 81) (width 0.6) (layer "F.Cu") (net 11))
 (segment (start 54.96 94.335) (end 53.26 92.635) (width 0.6) (layer "F.Cu") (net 11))
 (segment (start 69.204164 112.115) (end 67.64 112.115) (width 0.6) (layer "F.Cu") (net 11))
 (segment (start 90.22 77.72) (end 87.46 80.48) (width 0.6) (layer "F.Cu") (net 11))
 (segment (start 90.22 75) (end 90.22 77.72) (width 0.6) (layer "F.Cu") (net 11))
 (segment (start 87.46 81) (end 87.46 93.859164) (width 0.6) (layer "F.Cu") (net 11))
 (segment (start 67.64 112.115) (end 54.96 99.435) (width 0.6) (layer "F.Cu") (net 11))
 (segment (start 54.96 99.435) (end 54.96 94.335) (width 0.6) (layer "F.Cu") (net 11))
 (segment (start 53.755836 113.315) (end 51.56 111.119164) (width 0.6) (layer "F.Cu") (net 12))
 (segment (start 92.76 75) (end 92.76 78.24) (width 0.6) (layer "F.Cu") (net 12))
 (segment (start 51.56 91.795) (end 53.26 90.095) (width 0.6) (layer "F.Cu") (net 12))
 (segment (start 90 93.01622) (end 69.70122 113.315) (width 0.6) (layer "F.Cu") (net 12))
 (segment (start 90 81) (end 90 93.01622) (width 0.6) (layer "F.Cu") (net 12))
 (segment (start 69.70122 113.315) (end 53.755836 113.315) (width 0.6) (layer "F.Cu") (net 12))
 (segment (start 92.76 78.24) (end 90 81) (width 0.6) (layer "F.Cu") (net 12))
 (segment (start 51.56 111.119164) (end 51.56 91.795) (width 0.6) (layer "F.Cu") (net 12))
 (segment (start 86.265 55.21) (end 82.598528 58.876472) (width 0.6) (layer "F.Cu") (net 6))
 (segment (start 81.46 43.475) (end 86.265 48.28) (width 0.6) (layer "F.Cu") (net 6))
 (segment (start 75.4 59.177944) (end 75.4 85.735) (width 0.6) (layer "F.Cu") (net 6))
 (segment (start 75.4 85.735) (end 68.5 92.635) (width 0.6) (layer "F.Cu") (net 6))
 (segment (start 75.098528 58.876472) (end 75.4 59.177944) (width 0.6) (layer "F.Cu") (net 6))
 (segment (start 86.265 48.28) (end 86.265 55.21) (width 0.6) (layer "F.Cu") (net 6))
 (segment (start 82.598528 58.876472) (end 75.098528 58.876472) (width 0.6) (layer "F.Cu") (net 6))
 (segment (start 83.095584 60.076472) (end 77 60.076472) (width 0.6) (layer "F.Cu") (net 5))
 (segment (start 77 60.076472) (end 77 86.675) (width 0.6) (layer "F.Cu") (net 5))
 (segment (start 84 43.475) (end 87.465 46.94) (width 0.6) (layer "F.Cu") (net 5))
 (segment (start 87.465 46.94) (end 87.465 55.707056) (width 0.6) (layer "F.Cu") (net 5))
 (segment (start 87.465 55.707056) (end 83.095584 60.076472) (width 0.6) (layer "F.Cu") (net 5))
 (segment (start 77 86.675) (end 68.5 95.175) (width 0.6) (layer "F.Cu") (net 5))
 (segment (start 83.394112 61.475) (end 78.2 61.475) (width 0.6) (layer "F.Cu") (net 4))
 (segment (start 88.665 45.6) (end 88.665 56.204112) (width 0.6) (layer "F.Cu") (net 4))
 (segment (start 88.665 56.204112) (end 83.394112 61.475) (width 0.6) (layer "F.Cu") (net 4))
 (segment (start 78.2 61.475) (end 78.2 88.015) (width 0.6) (layer "F.Cu") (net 4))
 (segment (start 78.2 88.015) (end 68.5 97.715) (width 0.6) (layer "F.Cu") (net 4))
 (segment (start 86.54 43.475) (end 88.665 45.6) (width 0.6) (layer "F.Cu") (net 4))
 (segment (start 84.515 55.262944) (end 82.302944 57.475) (width 0.6) (layer "F.Cu") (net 9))
 (segment (start 74.2 84.395) (end 68.5 90.095) (width 0.6) (layer "F.Cu") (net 9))
 (segment (start 72 57.475) (end 74.2 59.675) (width 0.6) (layer "F.Cu") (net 9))
 (segment (start 82.302944 57.475) (end 72 57.475) (width 0.6) (layer "F.Cu") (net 9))
 (segment (start 74.2 59.675) (end 74.2 84.395) (width 0.6) (layer "F.Cu") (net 9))
 (segment (start 84.515 53.975) (end 84.515 55.262944) (width 0.6) (layer "F.Cu") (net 9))
 (segment (start 89.75 67.25) (end 85.15 67.25) (width 0.6) (layer "F.Cu") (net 7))
 (segment (start 79.4 73) (end 79.4 89.355) (width 0.6) (layer "F.Cu") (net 7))
 (segment (start 91.5 69) (end 89.75 67.25) (width 0.6) (layer "F.Cu") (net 7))
 (segment (start 79.4 89.355) (end 68.5 100.255) (width 0.6) (layer "F.Cu") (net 7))
 (segment (start 85.15 67.25) (end 79.4 73) (width 0.6) (layer "F.Cu") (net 7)))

